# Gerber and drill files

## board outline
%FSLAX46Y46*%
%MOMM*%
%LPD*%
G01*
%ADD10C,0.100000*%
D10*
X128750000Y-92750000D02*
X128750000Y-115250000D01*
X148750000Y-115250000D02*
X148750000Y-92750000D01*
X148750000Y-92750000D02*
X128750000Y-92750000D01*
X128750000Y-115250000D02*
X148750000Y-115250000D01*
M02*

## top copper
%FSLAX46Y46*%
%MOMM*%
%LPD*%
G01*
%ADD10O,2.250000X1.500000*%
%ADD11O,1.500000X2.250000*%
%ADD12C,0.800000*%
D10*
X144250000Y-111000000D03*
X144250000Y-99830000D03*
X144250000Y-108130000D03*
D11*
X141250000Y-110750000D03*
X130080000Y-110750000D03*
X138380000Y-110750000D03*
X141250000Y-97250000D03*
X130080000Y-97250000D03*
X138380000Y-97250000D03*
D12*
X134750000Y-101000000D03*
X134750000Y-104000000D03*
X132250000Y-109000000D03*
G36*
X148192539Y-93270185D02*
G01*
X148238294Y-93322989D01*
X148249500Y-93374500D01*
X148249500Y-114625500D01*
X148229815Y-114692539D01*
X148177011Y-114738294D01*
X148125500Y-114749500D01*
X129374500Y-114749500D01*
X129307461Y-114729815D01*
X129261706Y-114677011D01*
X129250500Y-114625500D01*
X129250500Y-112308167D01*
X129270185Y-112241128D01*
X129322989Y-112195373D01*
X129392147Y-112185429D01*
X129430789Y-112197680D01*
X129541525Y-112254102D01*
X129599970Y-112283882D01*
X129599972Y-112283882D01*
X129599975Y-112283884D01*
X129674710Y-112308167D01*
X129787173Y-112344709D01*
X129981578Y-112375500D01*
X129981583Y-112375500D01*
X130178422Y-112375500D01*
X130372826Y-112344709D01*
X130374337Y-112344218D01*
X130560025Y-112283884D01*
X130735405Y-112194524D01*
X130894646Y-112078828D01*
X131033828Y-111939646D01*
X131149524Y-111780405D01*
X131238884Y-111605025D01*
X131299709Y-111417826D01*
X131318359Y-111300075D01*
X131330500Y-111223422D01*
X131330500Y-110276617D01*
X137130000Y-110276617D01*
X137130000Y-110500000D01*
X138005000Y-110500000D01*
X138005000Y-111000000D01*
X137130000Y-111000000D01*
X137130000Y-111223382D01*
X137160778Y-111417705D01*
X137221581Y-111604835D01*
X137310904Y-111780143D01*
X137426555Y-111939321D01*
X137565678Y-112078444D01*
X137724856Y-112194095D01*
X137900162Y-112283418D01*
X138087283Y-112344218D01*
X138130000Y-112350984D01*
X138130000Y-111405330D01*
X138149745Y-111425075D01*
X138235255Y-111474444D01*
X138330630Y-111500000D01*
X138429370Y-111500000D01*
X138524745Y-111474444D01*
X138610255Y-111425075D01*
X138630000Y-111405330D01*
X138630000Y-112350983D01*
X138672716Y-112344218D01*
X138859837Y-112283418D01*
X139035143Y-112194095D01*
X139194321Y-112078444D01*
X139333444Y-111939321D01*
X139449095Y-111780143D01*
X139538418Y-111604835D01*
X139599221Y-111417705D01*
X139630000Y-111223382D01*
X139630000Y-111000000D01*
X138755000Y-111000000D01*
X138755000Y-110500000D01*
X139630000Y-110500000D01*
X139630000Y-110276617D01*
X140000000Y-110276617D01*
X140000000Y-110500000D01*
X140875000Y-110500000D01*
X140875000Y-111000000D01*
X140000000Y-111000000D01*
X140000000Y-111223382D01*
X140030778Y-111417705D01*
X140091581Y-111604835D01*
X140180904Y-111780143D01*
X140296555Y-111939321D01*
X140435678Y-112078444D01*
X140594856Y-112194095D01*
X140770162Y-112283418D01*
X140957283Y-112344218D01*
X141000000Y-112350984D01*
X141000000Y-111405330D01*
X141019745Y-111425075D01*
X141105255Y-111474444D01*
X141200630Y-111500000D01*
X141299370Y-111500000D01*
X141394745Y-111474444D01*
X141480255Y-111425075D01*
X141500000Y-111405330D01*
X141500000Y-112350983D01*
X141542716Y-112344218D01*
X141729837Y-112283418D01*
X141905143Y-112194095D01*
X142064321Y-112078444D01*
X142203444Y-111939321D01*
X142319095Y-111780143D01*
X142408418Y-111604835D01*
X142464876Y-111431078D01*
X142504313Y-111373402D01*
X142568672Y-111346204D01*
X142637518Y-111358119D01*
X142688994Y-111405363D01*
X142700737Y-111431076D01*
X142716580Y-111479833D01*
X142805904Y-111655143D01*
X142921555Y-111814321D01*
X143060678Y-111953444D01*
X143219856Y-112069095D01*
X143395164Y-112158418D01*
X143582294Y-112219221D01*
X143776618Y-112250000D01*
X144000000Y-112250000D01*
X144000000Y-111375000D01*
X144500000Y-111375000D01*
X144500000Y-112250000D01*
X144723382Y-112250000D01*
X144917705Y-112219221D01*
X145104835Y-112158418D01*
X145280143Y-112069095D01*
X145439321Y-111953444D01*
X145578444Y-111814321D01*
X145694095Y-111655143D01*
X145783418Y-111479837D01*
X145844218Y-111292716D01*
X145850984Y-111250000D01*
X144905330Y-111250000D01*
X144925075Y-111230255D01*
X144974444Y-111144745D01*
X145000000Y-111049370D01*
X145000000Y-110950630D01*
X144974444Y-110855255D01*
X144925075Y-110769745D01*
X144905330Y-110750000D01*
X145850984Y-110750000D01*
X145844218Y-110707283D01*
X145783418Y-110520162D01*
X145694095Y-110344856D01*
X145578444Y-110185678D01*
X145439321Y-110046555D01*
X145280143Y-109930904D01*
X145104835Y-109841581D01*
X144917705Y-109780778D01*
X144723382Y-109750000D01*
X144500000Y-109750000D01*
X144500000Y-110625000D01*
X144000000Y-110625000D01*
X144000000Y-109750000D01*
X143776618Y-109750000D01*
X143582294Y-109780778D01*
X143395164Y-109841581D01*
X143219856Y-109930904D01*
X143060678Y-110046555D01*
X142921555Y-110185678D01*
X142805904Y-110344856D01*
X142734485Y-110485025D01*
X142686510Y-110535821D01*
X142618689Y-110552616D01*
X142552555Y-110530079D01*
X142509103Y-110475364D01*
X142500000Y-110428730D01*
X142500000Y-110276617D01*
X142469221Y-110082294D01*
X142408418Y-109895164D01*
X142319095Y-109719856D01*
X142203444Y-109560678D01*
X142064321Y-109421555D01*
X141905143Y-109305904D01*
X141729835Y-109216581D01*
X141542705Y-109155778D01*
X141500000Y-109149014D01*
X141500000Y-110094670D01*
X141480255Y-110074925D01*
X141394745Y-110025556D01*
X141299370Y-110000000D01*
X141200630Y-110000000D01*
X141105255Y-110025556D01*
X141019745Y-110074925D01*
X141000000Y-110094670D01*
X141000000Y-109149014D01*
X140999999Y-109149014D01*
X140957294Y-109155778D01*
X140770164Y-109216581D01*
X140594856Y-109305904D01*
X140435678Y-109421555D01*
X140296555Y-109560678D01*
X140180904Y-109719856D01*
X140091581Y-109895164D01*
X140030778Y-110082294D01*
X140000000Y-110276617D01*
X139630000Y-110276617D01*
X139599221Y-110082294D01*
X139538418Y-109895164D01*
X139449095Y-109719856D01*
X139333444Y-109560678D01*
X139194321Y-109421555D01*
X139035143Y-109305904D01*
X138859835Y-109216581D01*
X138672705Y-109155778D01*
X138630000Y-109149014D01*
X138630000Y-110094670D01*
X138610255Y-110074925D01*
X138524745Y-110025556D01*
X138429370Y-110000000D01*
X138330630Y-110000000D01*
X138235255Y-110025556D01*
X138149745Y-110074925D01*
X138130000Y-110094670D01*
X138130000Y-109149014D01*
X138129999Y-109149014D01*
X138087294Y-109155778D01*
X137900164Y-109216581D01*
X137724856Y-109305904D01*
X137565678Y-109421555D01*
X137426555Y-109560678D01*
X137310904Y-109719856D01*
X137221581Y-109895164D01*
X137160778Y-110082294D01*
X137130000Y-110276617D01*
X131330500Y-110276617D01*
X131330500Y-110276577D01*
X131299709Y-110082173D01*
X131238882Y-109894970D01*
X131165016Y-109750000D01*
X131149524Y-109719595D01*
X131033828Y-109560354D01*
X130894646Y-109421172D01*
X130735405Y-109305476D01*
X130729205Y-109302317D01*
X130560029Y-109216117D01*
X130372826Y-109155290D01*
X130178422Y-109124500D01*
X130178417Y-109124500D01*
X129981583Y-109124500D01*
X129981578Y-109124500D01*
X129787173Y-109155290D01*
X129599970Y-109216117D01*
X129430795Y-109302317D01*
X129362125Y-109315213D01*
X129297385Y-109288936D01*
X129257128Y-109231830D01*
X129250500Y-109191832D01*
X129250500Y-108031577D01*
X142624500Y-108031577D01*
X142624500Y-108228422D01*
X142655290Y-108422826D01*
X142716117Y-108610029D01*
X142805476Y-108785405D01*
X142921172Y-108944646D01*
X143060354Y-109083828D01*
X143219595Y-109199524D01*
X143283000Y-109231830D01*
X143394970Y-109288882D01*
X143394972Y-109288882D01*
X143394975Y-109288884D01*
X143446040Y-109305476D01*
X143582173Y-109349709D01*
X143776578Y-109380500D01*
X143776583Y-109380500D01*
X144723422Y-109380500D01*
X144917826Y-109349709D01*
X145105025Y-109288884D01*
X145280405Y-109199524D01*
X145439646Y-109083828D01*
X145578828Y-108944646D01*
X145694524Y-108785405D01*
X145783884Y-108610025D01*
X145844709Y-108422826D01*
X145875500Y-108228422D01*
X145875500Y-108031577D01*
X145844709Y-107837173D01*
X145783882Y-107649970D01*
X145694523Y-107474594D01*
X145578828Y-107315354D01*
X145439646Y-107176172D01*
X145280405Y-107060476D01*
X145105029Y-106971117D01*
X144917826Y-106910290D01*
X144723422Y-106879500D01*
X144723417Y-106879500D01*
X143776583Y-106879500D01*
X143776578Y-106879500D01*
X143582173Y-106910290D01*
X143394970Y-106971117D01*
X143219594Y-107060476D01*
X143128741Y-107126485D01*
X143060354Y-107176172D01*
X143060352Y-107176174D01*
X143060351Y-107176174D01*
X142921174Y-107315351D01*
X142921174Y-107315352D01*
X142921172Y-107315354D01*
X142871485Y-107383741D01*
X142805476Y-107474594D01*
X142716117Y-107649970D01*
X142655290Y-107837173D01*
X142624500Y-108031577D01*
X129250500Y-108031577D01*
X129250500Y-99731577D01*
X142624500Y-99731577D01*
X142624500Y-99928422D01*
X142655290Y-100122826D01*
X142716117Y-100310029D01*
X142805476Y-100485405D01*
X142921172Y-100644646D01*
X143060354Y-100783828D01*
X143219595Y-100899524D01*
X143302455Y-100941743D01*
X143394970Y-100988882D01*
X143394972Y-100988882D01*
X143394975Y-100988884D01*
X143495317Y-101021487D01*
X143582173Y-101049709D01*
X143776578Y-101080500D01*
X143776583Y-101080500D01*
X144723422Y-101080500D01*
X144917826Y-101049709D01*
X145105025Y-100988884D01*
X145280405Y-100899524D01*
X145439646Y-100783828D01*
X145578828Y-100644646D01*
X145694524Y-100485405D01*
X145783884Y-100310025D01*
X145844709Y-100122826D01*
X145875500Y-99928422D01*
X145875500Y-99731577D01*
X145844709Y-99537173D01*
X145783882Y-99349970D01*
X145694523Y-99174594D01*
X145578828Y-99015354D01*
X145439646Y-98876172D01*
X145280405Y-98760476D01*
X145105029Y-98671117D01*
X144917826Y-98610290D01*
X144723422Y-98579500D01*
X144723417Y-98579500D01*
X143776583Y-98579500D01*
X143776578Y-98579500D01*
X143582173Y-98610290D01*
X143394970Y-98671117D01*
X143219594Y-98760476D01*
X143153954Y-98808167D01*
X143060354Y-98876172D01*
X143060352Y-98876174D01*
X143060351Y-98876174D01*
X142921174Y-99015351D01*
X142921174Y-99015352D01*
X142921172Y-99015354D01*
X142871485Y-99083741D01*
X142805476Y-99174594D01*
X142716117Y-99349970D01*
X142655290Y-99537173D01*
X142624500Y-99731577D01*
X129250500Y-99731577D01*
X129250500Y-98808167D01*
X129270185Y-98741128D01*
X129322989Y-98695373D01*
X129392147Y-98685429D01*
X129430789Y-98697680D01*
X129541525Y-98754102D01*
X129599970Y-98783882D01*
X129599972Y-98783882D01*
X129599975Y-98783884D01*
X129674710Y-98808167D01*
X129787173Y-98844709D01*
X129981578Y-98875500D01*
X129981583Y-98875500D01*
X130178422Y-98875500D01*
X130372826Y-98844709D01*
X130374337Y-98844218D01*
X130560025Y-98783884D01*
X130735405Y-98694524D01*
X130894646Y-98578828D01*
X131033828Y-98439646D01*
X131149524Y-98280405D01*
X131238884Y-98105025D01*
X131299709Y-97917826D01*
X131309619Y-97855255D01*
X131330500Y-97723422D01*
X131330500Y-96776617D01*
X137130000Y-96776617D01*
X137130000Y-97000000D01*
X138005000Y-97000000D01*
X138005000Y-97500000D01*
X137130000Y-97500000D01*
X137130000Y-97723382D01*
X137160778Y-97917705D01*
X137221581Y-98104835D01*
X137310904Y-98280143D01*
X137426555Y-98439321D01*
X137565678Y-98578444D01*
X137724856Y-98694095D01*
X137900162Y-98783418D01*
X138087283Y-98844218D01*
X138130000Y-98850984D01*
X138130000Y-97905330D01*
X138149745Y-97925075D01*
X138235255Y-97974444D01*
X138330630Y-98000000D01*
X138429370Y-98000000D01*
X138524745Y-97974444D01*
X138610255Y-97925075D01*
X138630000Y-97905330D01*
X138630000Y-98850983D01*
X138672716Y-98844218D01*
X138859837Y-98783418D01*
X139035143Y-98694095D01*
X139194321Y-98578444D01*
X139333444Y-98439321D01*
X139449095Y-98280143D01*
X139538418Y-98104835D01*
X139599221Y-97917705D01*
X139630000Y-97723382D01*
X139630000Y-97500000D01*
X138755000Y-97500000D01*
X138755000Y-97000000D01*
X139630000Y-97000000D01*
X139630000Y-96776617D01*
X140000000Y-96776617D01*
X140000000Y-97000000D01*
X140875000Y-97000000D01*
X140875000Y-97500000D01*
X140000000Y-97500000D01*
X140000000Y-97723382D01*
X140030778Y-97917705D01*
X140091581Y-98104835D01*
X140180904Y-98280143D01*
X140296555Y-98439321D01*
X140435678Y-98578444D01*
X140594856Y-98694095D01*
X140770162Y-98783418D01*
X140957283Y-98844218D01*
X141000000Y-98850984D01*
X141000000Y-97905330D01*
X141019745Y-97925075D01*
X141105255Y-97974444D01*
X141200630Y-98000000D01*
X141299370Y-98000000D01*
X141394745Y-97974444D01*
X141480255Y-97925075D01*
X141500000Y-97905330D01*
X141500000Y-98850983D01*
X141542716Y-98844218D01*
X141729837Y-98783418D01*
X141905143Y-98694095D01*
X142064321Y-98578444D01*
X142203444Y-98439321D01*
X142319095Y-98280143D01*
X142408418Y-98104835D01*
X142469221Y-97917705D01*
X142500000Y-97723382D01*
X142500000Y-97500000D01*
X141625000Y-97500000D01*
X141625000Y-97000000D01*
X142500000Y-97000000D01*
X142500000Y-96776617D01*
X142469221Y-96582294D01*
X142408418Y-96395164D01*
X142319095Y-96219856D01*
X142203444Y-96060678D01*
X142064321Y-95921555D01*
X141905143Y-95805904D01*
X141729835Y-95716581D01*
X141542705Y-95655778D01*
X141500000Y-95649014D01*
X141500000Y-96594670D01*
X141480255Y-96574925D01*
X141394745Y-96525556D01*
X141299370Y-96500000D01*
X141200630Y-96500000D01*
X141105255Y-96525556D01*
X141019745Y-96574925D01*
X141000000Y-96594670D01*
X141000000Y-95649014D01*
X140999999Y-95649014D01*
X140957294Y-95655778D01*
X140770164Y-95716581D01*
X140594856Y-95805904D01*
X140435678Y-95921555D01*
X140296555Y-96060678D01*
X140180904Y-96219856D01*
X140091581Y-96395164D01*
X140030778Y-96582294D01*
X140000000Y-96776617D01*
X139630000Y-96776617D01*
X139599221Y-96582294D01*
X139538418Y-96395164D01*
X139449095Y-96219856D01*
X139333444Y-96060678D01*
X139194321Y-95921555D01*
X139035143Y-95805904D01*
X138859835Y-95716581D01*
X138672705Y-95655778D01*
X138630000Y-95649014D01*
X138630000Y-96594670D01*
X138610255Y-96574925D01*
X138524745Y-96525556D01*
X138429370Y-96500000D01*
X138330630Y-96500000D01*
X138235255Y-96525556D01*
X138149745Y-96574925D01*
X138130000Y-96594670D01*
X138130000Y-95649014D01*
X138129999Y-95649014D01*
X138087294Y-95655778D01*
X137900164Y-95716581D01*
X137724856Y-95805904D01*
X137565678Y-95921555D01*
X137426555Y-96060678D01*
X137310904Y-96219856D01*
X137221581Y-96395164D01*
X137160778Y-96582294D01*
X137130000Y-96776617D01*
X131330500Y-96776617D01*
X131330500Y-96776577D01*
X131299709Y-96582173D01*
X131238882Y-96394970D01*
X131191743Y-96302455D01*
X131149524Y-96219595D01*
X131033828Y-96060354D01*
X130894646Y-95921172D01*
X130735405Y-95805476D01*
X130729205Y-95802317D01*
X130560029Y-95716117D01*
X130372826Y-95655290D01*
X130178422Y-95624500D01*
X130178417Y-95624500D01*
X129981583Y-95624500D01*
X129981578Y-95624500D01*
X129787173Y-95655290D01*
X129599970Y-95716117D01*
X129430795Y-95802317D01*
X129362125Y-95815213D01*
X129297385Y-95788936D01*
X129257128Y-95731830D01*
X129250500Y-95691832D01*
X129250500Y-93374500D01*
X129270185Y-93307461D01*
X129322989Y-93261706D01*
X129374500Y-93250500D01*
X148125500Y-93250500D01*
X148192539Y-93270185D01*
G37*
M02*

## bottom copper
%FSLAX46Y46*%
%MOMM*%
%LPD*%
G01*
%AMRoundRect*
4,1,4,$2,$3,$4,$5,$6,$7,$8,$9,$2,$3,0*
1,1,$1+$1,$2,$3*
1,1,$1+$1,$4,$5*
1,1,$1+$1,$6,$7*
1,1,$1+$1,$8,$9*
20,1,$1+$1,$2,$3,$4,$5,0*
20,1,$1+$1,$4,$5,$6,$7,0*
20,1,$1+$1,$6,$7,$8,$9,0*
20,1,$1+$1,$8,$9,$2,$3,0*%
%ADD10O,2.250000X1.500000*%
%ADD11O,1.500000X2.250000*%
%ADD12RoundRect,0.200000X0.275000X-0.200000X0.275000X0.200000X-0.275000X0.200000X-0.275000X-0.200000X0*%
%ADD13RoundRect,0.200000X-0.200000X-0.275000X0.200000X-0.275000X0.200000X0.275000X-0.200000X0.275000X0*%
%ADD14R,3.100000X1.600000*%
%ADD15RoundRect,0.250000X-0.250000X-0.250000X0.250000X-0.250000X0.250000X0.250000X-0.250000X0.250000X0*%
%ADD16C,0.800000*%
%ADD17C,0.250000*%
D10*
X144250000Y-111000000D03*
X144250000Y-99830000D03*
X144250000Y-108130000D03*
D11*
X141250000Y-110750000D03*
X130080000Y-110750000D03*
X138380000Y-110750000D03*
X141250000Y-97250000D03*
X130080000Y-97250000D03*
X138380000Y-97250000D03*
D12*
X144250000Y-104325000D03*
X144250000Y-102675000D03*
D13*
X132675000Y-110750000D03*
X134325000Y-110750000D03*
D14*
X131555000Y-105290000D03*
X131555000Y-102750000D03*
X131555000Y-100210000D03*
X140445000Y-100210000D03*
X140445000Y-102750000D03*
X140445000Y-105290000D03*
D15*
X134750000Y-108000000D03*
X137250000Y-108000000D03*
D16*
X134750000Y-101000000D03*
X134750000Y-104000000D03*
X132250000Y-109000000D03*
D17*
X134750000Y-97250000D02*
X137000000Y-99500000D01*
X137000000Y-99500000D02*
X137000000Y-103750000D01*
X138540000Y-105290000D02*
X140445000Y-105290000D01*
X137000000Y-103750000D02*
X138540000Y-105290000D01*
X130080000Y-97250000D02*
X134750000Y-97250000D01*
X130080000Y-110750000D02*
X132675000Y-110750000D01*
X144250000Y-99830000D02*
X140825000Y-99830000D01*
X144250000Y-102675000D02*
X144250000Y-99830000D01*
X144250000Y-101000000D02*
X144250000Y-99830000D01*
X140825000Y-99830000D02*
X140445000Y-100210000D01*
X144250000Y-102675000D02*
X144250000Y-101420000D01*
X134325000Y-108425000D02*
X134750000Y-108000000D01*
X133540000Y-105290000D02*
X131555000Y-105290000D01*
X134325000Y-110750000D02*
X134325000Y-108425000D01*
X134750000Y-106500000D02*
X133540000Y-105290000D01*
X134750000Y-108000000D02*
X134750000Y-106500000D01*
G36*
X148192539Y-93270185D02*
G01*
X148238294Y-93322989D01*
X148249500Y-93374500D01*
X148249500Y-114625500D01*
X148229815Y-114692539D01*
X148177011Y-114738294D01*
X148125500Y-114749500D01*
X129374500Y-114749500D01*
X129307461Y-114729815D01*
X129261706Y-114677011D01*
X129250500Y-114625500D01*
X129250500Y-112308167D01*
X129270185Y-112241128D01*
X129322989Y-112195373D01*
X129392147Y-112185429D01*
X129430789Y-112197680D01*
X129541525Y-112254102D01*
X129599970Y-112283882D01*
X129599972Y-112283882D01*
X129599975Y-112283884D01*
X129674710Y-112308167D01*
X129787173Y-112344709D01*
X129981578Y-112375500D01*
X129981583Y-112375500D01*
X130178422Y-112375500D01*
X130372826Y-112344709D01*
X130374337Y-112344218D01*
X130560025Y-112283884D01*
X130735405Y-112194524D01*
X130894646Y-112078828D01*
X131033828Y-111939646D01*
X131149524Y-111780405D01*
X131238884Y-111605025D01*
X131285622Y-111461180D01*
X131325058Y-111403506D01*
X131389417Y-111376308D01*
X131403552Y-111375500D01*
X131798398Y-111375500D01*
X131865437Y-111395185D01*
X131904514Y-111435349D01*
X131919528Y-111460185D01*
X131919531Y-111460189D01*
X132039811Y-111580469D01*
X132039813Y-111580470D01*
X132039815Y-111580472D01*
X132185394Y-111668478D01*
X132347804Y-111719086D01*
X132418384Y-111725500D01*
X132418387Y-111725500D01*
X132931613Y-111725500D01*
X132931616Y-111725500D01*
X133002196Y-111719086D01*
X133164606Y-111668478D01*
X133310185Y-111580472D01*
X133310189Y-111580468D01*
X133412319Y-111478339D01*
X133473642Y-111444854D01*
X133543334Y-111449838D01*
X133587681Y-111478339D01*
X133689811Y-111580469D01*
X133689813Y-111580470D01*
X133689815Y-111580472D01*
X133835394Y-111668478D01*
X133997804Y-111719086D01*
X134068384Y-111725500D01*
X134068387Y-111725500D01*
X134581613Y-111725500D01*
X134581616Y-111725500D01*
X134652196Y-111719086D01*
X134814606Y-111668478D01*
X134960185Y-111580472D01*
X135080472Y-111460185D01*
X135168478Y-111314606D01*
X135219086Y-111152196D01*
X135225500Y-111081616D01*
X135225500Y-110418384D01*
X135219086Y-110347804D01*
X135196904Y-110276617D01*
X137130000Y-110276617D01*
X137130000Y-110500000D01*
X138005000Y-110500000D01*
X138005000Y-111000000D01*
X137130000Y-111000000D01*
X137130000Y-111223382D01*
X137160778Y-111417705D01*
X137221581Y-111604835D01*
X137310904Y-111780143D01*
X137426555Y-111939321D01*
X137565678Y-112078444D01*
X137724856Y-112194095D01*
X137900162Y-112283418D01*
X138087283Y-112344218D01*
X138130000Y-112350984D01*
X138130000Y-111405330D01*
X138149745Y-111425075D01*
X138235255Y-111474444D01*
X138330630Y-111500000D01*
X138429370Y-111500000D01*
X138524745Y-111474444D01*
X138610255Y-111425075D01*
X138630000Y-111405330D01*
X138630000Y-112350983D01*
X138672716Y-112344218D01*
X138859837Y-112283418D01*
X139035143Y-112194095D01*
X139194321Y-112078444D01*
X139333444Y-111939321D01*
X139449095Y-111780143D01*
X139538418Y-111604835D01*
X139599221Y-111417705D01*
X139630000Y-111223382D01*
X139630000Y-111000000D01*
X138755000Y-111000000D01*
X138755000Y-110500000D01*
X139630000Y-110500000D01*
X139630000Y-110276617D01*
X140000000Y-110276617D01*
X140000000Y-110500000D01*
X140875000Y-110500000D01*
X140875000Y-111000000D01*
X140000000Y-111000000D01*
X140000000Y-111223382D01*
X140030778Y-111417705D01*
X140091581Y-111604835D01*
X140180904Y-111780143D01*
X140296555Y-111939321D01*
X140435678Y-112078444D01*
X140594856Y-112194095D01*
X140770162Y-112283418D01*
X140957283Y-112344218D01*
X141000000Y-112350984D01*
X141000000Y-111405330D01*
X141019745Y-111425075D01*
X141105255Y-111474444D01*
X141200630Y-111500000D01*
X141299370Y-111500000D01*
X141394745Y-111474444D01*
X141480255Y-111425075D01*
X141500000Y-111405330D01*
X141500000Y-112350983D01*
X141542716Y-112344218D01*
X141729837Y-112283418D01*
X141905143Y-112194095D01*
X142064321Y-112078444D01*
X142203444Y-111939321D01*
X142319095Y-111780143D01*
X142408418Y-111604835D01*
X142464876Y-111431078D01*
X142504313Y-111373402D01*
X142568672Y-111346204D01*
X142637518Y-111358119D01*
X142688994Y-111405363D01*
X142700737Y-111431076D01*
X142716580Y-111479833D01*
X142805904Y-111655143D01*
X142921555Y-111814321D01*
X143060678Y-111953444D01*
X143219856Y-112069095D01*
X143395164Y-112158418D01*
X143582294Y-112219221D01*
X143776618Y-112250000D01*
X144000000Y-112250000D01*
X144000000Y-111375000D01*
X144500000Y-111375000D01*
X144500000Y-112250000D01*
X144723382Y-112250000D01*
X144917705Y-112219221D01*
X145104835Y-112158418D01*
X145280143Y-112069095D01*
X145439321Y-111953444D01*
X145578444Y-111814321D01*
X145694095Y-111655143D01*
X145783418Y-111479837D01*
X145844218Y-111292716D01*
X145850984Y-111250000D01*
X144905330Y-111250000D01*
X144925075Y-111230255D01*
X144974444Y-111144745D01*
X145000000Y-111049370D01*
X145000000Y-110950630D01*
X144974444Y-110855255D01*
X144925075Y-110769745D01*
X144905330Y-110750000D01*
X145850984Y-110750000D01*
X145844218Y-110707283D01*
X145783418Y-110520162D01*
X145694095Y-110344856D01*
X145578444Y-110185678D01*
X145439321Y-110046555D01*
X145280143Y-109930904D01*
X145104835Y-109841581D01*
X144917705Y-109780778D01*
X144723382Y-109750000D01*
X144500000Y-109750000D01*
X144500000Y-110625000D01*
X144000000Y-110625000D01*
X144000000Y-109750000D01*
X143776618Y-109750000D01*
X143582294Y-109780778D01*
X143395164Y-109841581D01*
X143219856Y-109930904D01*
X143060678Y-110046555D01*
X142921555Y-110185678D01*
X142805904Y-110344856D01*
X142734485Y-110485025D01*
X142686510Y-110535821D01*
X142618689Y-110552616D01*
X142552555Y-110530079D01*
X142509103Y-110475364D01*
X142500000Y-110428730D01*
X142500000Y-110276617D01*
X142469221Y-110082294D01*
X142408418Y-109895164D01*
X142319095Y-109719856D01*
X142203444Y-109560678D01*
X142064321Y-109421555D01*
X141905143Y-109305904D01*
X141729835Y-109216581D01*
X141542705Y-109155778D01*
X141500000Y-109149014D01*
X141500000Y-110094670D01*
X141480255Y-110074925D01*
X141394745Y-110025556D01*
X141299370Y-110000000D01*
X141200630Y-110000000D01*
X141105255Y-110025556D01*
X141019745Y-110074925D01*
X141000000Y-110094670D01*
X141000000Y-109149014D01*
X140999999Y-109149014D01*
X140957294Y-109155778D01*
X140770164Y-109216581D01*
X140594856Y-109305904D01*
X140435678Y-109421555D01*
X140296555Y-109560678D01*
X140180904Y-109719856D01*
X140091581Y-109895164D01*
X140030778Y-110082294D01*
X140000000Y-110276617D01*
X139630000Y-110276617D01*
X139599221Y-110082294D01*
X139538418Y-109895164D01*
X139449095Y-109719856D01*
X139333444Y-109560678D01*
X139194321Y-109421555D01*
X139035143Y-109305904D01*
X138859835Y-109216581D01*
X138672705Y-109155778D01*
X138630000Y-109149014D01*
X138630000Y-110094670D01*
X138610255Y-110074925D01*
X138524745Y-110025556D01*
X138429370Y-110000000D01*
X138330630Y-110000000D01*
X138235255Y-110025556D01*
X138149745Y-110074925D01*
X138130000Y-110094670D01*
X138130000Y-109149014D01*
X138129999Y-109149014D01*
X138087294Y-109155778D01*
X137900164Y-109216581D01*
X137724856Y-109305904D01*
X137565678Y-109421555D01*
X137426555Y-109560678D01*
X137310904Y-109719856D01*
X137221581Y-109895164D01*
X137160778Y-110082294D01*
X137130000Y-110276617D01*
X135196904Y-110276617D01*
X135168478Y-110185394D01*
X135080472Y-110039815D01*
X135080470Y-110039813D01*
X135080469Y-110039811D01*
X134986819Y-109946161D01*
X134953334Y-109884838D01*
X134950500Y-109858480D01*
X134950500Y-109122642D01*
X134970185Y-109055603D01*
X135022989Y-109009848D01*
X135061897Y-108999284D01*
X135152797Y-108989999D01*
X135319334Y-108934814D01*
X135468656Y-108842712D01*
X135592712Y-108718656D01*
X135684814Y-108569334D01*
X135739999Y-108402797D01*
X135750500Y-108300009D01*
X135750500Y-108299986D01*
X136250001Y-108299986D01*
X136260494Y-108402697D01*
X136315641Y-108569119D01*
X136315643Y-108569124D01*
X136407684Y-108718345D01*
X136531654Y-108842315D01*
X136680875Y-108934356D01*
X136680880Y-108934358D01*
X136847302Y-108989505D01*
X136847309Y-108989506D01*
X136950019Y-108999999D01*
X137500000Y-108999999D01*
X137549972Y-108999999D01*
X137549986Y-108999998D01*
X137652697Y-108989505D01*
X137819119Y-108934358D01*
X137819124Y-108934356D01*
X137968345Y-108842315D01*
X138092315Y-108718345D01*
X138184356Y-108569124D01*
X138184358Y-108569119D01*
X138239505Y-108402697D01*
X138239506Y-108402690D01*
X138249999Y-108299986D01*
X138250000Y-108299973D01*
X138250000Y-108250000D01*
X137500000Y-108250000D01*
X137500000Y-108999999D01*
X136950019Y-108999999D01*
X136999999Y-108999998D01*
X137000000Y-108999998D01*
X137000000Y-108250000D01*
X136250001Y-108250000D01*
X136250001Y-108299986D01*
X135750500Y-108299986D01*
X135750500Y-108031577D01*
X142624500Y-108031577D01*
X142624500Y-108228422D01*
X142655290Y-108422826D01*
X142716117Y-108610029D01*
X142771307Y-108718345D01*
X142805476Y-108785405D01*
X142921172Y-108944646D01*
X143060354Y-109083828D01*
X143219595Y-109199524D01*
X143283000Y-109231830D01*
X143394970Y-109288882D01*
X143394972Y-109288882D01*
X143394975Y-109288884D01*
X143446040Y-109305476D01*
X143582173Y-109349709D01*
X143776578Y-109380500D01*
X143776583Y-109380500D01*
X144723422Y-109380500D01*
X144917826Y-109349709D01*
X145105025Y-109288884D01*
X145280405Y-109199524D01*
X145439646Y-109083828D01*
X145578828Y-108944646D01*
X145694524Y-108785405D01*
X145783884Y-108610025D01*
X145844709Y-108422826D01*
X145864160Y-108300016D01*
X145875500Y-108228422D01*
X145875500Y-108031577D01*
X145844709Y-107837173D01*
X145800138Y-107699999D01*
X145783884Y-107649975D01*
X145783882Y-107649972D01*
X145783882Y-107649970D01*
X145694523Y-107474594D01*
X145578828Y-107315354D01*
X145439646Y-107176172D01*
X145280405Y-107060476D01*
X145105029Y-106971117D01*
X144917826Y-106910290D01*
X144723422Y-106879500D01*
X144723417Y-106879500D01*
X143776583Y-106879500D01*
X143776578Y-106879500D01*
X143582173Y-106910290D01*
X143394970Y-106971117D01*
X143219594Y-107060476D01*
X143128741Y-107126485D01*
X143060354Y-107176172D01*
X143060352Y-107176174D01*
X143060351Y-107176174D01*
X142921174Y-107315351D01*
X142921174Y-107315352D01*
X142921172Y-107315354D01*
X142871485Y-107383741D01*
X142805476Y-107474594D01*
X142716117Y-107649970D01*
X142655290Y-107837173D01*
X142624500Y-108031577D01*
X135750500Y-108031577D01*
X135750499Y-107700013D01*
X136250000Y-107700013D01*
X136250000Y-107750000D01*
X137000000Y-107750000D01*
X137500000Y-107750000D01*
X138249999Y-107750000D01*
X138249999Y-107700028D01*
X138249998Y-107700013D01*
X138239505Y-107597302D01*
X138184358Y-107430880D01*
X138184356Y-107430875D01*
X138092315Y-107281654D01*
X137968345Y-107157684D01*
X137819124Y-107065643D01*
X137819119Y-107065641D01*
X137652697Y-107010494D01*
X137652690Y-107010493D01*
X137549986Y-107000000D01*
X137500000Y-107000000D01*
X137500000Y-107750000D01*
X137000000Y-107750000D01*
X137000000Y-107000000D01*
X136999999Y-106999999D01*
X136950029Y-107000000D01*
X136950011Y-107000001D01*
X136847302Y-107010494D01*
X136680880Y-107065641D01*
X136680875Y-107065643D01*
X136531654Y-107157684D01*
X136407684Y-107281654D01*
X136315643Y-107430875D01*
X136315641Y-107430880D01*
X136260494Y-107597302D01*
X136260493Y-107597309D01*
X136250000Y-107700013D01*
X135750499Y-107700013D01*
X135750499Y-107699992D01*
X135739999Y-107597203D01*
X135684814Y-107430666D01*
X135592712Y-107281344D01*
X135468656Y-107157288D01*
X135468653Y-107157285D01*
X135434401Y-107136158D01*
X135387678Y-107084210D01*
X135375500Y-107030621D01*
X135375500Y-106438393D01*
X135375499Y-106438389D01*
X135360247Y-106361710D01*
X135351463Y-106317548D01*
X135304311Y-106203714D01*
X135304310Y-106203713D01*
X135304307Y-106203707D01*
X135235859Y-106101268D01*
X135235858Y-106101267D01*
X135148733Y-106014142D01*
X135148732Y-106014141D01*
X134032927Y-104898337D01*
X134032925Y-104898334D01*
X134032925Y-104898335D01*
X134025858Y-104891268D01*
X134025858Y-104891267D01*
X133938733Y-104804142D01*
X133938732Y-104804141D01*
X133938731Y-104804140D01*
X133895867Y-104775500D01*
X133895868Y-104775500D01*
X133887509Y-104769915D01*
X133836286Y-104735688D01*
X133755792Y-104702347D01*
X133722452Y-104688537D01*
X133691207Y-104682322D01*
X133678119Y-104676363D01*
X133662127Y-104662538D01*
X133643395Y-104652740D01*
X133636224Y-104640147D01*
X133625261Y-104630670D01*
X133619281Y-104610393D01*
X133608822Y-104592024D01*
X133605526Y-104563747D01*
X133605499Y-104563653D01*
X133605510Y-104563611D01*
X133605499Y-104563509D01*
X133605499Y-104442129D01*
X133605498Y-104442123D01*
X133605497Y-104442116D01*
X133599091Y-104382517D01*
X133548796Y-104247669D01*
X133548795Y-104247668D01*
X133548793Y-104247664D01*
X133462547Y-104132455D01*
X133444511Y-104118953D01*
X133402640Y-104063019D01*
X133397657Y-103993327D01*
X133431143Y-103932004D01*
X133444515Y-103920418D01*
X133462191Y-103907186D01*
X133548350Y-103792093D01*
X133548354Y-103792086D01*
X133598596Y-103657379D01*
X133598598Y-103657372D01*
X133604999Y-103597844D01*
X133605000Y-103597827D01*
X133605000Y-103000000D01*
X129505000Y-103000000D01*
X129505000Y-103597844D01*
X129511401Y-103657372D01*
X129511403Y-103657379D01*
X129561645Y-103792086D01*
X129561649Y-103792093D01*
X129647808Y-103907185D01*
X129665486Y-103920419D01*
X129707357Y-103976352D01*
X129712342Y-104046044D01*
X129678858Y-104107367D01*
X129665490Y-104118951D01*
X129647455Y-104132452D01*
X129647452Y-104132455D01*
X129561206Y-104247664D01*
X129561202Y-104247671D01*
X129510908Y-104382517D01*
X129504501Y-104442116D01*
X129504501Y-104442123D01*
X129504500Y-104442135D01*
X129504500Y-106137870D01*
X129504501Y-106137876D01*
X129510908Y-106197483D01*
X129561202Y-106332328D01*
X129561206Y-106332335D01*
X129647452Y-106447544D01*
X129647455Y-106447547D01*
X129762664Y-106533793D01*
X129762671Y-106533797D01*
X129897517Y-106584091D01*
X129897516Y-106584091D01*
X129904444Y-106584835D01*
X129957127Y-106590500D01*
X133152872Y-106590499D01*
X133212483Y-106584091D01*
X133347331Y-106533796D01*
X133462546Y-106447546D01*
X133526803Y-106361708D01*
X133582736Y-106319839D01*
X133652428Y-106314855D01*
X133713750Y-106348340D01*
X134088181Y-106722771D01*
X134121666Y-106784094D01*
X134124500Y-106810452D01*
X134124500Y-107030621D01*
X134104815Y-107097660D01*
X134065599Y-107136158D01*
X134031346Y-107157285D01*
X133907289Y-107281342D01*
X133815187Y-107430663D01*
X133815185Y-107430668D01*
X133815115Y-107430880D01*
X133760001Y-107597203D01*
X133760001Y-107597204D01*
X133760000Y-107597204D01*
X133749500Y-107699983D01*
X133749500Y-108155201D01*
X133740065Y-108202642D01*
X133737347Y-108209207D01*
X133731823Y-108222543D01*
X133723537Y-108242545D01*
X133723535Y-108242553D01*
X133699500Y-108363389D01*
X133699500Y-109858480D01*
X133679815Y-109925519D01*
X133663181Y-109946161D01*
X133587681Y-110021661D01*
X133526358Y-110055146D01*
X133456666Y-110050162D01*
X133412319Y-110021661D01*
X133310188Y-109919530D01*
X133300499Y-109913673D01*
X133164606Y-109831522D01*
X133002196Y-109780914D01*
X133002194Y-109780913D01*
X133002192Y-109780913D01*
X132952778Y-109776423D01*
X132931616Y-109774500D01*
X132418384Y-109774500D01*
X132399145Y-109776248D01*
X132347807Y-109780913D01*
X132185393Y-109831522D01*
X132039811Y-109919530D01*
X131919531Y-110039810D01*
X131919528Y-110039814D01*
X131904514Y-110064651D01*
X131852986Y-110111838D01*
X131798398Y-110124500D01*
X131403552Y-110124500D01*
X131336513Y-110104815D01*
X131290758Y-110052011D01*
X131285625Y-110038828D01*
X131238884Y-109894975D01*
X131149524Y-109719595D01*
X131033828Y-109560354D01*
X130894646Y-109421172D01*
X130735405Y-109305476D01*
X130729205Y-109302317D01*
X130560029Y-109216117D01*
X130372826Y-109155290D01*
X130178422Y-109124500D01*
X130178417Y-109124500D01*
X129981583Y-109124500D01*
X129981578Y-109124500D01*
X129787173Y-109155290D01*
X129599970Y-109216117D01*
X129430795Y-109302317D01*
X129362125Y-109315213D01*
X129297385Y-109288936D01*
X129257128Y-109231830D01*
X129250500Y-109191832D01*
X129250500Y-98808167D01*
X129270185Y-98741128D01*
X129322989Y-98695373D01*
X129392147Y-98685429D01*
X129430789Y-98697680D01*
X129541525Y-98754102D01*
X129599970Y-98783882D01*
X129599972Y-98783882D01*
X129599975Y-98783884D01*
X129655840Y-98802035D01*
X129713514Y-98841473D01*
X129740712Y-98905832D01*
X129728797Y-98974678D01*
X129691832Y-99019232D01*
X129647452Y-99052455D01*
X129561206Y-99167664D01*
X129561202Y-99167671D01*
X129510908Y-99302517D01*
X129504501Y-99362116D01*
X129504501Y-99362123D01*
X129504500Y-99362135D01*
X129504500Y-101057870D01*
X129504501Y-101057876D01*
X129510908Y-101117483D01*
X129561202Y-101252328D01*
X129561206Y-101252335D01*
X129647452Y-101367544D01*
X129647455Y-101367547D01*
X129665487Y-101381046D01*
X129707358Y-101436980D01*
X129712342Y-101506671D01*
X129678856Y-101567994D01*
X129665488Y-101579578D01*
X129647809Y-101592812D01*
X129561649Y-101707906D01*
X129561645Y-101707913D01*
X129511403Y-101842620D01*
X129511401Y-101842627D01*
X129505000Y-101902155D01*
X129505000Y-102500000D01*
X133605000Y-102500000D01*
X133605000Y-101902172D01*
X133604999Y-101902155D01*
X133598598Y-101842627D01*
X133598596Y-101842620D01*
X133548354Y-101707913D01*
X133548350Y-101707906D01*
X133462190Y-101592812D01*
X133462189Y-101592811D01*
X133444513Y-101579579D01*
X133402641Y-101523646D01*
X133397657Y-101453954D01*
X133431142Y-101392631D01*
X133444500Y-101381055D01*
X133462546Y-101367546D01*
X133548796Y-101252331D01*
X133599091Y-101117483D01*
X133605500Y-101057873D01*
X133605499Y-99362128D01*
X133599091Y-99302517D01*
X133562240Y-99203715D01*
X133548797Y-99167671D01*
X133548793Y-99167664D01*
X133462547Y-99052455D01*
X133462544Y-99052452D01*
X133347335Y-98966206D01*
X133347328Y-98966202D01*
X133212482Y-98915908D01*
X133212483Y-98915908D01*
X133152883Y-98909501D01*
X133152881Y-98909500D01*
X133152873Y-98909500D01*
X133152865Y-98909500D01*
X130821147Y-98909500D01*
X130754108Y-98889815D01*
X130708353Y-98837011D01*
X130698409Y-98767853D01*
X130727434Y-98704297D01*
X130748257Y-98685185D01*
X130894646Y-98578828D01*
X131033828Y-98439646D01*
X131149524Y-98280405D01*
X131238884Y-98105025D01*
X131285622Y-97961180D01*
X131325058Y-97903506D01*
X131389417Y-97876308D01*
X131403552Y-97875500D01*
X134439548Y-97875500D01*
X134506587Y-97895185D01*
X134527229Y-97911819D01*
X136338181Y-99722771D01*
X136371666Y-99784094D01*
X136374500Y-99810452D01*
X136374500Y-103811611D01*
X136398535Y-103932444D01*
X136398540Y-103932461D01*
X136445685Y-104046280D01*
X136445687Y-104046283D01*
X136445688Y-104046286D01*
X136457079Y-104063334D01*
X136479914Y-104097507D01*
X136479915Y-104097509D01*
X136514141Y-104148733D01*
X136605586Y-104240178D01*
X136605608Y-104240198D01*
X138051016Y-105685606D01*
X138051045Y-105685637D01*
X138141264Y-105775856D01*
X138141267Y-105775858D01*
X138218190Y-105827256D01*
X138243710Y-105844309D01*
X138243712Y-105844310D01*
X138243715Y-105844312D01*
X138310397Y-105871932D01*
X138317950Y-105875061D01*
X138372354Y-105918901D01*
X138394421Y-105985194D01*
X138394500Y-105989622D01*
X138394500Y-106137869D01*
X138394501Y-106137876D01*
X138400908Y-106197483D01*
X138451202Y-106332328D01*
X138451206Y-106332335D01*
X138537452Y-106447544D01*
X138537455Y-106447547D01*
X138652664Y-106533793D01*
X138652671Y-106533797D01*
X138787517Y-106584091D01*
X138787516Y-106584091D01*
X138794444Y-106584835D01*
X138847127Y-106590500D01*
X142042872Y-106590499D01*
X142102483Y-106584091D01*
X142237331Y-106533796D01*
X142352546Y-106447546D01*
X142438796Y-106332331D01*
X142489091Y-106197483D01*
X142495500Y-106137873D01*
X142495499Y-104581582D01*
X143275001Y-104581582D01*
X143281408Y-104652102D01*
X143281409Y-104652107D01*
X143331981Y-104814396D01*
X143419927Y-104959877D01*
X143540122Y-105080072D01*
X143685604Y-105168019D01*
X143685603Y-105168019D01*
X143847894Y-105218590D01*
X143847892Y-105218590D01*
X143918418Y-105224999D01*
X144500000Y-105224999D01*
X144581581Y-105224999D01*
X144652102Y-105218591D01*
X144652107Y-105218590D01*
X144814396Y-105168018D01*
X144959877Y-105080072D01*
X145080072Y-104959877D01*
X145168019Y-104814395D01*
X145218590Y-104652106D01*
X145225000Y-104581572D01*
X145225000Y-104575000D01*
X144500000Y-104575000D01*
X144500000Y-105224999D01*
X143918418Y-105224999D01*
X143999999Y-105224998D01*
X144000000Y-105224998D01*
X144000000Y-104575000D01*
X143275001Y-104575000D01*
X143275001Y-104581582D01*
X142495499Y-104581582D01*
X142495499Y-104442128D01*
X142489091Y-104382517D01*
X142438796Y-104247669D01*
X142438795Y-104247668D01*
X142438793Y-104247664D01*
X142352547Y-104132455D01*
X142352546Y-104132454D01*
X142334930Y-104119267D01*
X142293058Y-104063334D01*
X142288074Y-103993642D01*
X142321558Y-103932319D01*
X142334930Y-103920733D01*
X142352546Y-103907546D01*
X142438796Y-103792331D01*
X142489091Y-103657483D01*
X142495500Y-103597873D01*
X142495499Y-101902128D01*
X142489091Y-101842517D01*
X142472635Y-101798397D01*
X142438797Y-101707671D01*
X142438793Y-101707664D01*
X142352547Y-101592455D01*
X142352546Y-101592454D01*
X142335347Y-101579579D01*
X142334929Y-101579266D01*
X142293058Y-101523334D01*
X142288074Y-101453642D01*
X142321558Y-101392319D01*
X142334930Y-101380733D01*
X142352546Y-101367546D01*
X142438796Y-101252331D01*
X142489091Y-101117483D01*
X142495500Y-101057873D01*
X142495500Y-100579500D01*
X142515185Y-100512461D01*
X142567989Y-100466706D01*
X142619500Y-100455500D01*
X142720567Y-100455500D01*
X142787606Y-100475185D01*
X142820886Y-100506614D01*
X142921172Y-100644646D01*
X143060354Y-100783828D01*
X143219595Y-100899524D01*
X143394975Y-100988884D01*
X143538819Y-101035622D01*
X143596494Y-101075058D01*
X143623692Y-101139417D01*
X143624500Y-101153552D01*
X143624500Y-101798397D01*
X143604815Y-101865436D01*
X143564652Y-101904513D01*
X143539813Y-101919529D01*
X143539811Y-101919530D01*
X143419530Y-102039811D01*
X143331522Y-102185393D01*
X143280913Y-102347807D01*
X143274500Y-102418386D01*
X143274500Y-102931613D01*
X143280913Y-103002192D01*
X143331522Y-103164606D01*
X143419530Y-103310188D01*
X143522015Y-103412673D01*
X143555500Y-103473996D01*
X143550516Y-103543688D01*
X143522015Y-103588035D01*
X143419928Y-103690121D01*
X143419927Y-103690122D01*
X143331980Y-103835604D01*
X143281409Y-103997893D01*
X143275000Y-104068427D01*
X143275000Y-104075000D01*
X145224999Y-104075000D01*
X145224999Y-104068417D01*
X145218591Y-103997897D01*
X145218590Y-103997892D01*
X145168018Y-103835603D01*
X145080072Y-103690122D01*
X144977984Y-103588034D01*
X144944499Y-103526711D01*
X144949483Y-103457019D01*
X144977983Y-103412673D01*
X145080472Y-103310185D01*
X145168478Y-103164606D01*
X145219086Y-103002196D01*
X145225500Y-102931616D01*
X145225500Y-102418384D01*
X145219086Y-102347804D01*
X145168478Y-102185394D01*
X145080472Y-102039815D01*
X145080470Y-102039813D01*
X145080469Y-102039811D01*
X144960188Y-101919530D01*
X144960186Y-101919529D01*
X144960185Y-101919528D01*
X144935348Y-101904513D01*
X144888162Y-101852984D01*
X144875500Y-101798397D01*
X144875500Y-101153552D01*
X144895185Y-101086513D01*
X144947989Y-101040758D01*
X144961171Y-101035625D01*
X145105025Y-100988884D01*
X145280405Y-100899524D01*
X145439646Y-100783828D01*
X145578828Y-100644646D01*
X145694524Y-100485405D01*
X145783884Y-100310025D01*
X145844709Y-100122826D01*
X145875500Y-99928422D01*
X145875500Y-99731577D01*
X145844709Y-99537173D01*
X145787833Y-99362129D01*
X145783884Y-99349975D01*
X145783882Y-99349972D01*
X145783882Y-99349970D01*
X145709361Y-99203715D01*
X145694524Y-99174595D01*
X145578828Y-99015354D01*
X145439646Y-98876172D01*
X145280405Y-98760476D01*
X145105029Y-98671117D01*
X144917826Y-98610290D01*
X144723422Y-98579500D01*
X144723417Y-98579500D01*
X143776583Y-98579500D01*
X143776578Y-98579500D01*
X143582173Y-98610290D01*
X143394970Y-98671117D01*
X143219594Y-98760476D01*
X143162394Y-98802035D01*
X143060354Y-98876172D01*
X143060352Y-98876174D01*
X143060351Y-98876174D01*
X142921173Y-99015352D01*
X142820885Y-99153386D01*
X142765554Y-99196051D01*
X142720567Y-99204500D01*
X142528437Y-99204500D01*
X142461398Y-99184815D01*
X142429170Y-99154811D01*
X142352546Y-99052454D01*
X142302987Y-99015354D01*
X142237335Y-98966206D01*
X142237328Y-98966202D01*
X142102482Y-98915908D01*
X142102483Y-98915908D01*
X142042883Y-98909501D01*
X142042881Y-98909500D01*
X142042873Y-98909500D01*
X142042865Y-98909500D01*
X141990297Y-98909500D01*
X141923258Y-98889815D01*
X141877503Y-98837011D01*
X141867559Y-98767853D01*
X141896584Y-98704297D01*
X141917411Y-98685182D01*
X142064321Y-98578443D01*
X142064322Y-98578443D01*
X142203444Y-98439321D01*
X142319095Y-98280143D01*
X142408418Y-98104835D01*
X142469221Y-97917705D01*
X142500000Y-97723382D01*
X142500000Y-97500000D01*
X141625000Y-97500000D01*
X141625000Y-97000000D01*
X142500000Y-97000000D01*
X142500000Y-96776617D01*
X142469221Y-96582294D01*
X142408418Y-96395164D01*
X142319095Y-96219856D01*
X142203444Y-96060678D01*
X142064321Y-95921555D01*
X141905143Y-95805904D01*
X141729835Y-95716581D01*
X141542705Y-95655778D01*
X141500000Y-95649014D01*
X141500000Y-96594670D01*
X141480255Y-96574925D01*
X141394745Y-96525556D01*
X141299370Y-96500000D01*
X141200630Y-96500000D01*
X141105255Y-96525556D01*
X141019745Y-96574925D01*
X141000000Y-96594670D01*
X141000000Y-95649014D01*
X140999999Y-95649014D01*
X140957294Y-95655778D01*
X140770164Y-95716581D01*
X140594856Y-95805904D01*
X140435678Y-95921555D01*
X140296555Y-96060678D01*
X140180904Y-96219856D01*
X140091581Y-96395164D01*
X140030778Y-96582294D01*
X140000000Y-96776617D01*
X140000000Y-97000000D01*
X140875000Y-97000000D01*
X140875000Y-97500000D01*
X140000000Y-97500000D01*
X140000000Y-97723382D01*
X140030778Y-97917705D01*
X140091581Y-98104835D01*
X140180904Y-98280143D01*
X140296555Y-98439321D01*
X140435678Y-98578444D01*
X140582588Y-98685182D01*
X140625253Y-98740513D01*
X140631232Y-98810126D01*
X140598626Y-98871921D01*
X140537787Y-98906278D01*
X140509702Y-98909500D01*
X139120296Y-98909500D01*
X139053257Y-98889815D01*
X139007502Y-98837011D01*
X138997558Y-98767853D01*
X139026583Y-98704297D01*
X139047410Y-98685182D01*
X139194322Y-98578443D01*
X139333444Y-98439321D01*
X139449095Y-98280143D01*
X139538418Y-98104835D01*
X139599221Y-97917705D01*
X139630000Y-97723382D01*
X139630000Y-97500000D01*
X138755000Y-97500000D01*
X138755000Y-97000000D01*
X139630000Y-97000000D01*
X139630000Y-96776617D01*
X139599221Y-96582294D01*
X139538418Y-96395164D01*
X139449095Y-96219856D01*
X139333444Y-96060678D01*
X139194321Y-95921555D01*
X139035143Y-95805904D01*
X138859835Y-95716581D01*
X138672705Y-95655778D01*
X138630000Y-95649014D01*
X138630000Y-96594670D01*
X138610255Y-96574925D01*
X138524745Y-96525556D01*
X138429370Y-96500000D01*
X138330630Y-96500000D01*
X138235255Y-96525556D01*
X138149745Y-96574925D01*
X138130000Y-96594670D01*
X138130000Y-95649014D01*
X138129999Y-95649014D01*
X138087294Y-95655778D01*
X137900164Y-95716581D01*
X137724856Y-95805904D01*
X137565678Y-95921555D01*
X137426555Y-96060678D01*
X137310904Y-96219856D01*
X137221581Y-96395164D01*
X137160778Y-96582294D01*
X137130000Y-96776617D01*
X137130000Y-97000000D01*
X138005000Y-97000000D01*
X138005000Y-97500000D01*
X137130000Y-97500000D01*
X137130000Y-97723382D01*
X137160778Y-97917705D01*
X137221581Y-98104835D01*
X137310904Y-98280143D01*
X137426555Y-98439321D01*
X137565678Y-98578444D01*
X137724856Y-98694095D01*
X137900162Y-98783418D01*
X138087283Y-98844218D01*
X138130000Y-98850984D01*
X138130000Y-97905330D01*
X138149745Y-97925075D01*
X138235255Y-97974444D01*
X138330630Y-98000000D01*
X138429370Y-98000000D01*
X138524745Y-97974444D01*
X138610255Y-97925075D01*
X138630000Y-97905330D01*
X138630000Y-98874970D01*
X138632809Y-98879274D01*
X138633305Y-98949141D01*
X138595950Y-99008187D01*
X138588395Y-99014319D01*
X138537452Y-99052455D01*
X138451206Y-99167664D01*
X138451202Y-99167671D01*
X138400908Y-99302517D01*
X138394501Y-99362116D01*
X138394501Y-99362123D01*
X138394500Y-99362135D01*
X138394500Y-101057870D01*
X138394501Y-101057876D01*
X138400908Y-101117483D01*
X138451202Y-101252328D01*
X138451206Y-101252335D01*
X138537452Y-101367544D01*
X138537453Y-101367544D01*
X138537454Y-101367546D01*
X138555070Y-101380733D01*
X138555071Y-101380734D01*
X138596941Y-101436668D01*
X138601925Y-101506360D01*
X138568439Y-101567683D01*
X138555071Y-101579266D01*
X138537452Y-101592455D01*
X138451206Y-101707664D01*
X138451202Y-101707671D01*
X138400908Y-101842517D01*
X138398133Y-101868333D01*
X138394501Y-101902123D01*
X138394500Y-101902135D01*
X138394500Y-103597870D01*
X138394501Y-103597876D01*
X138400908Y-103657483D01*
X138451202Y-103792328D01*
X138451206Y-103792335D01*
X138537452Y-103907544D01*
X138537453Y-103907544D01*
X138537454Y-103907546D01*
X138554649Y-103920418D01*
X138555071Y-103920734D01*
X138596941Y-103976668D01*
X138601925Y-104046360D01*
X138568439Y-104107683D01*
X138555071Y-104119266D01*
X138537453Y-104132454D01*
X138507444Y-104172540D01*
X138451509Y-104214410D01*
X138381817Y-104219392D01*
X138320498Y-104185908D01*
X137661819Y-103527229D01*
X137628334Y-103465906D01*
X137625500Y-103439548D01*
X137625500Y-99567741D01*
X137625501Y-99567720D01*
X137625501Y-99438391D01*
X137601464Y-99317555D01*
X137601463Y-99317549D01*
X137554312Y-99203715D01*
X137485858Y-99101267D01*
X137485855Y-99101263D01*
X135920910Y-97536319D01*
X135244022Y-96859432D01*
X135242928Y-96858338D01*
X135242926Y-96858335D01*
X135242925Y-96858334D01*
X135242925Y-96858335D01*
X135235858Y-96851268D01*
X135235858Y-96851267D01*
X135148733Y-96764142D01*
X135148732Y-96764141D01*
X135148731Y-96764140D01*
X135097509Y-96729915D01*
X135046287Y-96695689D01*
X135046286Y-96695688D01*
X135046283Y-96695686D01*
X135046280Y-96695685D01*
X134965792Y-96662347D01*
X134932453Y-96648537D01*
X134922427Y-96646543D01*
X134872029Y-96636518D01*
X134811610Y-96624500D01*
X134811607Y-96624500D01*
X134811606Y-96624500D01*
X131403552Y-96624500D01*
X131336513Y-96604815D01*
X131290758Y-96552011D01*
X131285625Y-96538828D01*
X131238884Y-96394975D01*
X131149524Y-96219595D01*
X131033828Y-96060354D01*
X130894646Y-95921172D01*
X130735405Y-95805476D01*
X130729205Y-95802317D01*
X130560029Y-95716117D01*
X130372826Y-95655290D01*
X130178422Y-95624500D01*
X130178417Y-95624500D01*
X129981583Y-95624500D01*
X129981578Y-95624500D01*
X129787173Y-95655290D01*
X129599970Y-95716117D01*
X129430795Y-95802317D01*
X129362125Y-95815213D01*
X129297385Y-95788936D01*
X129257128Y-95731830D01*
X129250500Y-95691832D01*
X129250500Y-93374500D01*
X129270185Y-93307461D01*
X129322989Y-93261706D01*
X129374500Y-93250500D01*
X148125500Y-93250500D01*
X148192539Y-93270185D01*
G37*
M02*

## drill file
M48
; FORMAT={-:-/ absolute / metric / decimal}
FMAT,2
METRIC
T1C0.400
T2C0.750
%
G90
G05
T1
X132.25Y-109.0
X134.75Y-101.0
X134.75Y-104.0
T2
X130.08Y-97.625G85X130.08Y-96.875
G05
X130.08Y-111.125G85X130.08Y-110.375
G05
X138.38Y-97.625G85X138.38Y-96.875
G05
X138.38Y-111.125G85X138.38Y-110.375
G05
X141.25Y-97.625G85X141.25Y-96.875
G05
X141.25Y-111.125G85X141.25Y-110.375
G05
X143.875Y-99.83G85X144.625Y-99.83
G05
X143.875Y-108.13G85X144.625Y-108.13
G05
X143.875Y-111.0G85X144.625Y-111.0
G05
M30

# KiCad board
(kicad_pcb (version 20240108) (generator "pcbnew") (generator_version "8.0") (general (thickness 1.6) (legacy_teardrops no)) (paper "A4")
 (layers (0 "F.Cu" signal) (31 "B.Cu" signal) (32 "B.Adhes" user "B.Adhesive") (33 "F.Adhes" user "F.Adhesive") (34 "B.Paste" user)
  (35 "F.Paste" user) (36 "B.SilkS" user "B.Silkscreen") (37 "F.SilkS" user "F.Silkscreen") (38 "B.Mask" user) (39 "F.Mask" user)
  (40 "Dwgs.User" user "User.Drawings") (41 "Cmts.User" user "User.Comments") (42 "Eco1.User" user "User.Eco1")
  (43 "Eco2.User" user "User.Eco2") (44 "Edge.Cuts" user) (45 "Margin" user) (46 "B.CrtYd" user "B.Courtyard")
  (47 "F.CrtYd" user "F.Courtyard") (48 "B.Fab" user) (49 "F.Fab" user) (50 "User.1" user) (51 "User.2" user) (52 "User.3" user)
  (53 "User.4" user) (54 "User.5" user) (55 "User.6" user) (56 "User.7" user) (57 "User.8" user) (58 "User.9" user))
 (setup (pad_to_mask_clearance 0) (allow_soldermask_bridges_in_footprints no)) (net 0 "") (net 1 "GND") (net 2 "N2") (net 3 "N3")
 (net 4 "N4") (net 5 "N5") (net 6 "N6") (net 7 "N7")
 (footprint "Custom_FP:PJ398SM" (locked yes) (layer "F.Cu") (at 144.25 104.75)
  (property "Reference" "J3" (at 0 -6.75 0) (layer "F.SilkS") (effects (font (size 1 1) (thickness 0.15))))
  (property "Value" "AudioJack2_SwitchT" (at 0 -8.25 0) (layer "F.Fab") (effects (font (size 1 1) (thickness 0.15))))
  (pad "S" thru_hole oval (at 0 6.25) (size 2.25 1.5) (drill oval 1.5 0.75) (layers "*.Cu" "*.Mask") (remove_unused_layers no) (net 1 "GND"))
  (pad "T" thru_hole oval (at 0 -4.92) (size 2.25 1.5) (drill oval 1.5 0.75) (layers "*.Cu" "*.Mask") (remove_unused_layers no) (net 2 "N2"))
  (pad "TN" thru_hole oval (at 0 3.38) (size 2.25 1.5) (drill oval 1.5 0.75) (layers "*.Cu" "*.Mask") (remove_unused_layers no) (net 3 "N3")))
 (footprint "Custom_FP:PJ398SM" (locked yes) (layer "F.Cu") (at 135 110.75 90)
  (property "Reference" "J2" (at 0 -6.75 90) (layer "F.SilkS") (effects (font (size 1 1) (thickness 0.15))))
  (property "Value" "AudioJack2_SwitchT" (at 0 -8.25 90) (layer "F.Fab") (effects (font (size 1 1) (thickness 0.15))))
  (pad "S" thru_hole oval (at 0 6.25 90) (size 2.25 1.5) (drill oval 1.5 0.75) (layers "*.Cu" "*.Mask") (remove_unused_layers no)
   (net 1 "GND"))
  (pad "T" thru_hole oval (at 0 -4.92 90) (size 2.25 1.5) (drill oval 1.5 0.75) (layers "*.Cu" "*.Mask") (remove_unused_layers no)
   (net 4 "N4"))
  (pad "TN" thru_hole oval (at 0 3.38 90) (size 2.25 1.5) (drill oval 1.5 0.75) (layers "*.Cu" "*.Mask") (remove_unused_layers no)
   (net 1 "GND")))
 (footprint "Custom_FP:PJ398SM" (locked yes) (layer "F.Cu") (at 135 97.25 90)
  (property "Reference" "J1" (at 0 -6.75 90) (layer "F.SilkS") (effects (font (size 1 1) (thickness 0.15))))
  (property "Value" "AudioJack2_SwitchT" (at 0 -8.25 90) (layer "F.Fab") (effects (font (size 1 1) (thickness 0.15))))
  (pad "S" thru_hole oval (at 0 6.25 90) (size 2.25 1.5) (drill oval 1.5 0.75) (layers "*.Cu" "*.Mask") (remove_unused_layers no)
   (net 1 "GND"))
  (pad "T" thru_hole oval (at 0 -4.92 90) (size 2.25 1.5) (drill oval 1.5 0.75) (layers "*.Cu" "*.Mask") (remove_unused_layers no)
   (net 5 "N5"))
  (pad "TN" thru_hole oval (at 0 3.38 90) (size 2.25 1.5) (drill oval 1.5 0.75) (layers "*.Cu" "*.Mask") (remove_unused_layers no)
   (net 1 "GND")))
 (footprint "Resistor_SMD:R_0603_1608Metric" (layer "B.Cu") (at 144.25 103.5 90)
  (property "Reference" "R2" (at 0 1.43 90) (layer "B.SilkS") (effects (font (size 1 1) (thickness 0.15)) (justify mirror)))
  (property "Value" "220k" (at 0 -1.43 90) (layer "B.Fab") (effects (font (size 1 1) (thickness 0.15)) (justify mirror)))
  (pad "1" smd roundrect (at -0.825 0 90) (size 0.8 0.95) (layers "B.Cu" "B.Paste" "B.Mask") (roundrect_rratio 0.25) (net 1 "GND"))
  (pad "2" smd roundrect (at 0.825 0 90) (size 0.8 0.95) (layers "B.Cu" "B.Paste" "B.Mask") (roundrect_rratio 0.25) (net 2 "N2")))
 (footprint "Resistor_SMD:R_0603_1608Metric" (layer "B.Cu") (at 133.5 110.75)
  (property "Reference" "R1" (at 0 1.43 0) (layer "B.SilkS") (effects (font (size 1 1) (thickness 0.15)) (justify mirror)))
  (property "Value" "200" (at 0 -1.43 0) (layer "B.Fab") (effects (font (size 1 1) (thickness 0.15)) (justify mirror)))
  (pad "1" smd roundrect (at -0.825 0) (size 0.8 0.95) (layers "B.Cu" "B.Paste" "B.Mask") (roundrect_rratio 0.25) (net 4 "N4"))
  (pad "2" smd roundrect (at 0.825 0) (size 0.8 0.95) (layers "B.Cu" "B.Paste" "B.Mask") (roundrect_rratio 0.25) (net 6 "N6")))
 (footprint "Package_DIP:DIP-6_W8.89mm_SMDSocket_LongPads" (layer "B.Cu") (at 136 102.75)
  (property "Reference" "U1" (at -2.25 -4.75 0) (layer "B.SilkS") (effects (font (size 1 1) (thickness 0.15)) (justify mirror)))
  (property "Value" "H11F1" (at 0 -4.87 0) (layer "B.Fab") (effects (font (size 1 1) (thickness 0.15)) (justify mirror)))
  (pad "1" smd rect (at -4.445 2.54) (size 3.1 1.6) (layers "B.Cu" "B.Paste" "B.Mask") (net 6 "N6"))
  (pad "2" smd rect (at -4.445 0) (size 3.1 1.6) (layers "B.Cu" "B.Paste" "B.Mask") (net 1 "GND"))
  (pad "3" smd rect (at -4.445 -2.54) (size 3.1 1.6) (layers "B.Cu" "B.Paste" "B.Mask") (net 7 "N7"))
  (pad "4" smd rect (at 4.445 -2.54) (size 3.1 1.6) (layers "B.Cu" "B.Paste" "B.Mask") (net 2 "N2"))
  (pad "5" smd rect (at 4.445 0) (size 3.1 1.6) (layers "B.Cu" "B.Paste" "B.Mask"))
  (pad "6" smd rect (at 4.445 2.54) (size 3.1 1.6) (layers "B.Cu" "B.Paste" "B.Mask") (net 5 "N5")))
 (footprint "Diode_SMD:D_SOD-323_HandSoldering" (layer "B.Cu") (at 136 108)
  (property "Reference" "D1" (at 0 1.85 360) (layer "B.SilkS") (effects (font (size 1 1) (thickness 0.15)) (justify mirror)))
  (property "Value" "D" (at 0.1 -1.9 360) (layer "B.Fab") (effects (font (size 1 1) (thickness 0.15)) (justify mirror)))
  (pad "1" smd roundrect (at -1.25 0) (size 1 1) (layers "B.Cu" "B.Paste" "B.Mask") (roundrect_rratio 0.25) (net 6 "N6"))
  (pad "2" smd roundrect (at 1.25 0) (size 1 1) (layers "B.Cu" "B.Paste" "B.Mask") (roundrect_rratio 0.25) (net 1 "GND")))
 (gr_line (start 128.75 92.75) (end 128.75 115.25) (stroke (width 0.1) (type default)) (layer "Edge.Cuts"))
 (gr_line (start 148.75 115.25) (end 148.75 92.75) (stroke (width 0.1) (type default)) (layer "Edge.Cuts"))
 (gr_line (start 148.75 92.75) (end 128.75 92.75) (stroke (width 0.1) (type default)) (layer "Edge.Cuts"))
 (gr_line (start 128.75 115.25) (end 148.75 115.25) (stroke (width 0.1) (type default)) (layer "Edge.Cuts"))
 (segment (start 134.75 97.25) (end 137 99.5) (width 0.25) (layer "B.Cu") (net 5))
 (segment (start 137 99.5) (end 137 103.75) (width 0.25) (layer "B.Cu") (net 5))
 (segment (start 138.54 105.29) (end 140.445 105.29) (width 0.25) (layer "B.Cu") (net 5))
 (segment (start 137 103.75) (end 138.54 105.29) (width 0.25) (layer "B.Cu") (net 5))
 (segment (start 130.08 97.25) (end 134.75 97.25) (width 0.25) (layer "B.Cu") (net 5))
 (via (at 134.75 101) (size 0.8) (drill 0.4) (layers "F.Cu" "B.Cu") (free yes) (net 1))
 (via (at 134.75 104) (size 0.8) (drill 0.4) (layers "F.Cu" "B.Cu") (free yes) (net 1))
 (via (at 132.25 109) (size 0.8) (drill 0.4) (layers "F.Cu" "B.Cu") (free yes) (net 1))
 (segment (start 130.08 110.75) (end 132.675 110.75) (width 0.25) (layer "B.Cu") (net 4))
 (segment (start 144.25 99.83) (end 140.825 99.83) (width 0.25) (layer "B.Cu") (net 2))
 (segment (start 144.25 102.675) (end 144.25 99.83) (width 0.25) (layer "B.Cu") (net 2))
 (segment (start 144.25 101) (end 144.25 99.83) (width 0.25) (layer "B.Cu") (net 2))
 (segment (start 140.825 99.83) (end 140.445 100.21) (width 0.25) (layer "B.Cu") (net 2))
 (segment (start 144.25 102.675) (end 144.25 101.42) (width 0.25) (layer "B.Cu") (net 2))
 (segment (start 134.325 108.425) (end 134.75 108) (width 0.25) (layer "B.Cu") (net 6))
 (segment (start 133.54 105.29) (end 131.555 105.29) (width 0.25) (layer "B.Cu") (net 6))
 (segment (start 134.325 110.75) (end 134.325 108.425) (width 0.25) (layer "B.Cu") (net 6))
 (segment (start 134.75 106.5) (end 133.54 105.29) (width 0.25) (layer "B.Cu") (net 6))
 (segment (start 134.75 108) (end 134.75 106.5) (width 0.25) (layer "B.Cu") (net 6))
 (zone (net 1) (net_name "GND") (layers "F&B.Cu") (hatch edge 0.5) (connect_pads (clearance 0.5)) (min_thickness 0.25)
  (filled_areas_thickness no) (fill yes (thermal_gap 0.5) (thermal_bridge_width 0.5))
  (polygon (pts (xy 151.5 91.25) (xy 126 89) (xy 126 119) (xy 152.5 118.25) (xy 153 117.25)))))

